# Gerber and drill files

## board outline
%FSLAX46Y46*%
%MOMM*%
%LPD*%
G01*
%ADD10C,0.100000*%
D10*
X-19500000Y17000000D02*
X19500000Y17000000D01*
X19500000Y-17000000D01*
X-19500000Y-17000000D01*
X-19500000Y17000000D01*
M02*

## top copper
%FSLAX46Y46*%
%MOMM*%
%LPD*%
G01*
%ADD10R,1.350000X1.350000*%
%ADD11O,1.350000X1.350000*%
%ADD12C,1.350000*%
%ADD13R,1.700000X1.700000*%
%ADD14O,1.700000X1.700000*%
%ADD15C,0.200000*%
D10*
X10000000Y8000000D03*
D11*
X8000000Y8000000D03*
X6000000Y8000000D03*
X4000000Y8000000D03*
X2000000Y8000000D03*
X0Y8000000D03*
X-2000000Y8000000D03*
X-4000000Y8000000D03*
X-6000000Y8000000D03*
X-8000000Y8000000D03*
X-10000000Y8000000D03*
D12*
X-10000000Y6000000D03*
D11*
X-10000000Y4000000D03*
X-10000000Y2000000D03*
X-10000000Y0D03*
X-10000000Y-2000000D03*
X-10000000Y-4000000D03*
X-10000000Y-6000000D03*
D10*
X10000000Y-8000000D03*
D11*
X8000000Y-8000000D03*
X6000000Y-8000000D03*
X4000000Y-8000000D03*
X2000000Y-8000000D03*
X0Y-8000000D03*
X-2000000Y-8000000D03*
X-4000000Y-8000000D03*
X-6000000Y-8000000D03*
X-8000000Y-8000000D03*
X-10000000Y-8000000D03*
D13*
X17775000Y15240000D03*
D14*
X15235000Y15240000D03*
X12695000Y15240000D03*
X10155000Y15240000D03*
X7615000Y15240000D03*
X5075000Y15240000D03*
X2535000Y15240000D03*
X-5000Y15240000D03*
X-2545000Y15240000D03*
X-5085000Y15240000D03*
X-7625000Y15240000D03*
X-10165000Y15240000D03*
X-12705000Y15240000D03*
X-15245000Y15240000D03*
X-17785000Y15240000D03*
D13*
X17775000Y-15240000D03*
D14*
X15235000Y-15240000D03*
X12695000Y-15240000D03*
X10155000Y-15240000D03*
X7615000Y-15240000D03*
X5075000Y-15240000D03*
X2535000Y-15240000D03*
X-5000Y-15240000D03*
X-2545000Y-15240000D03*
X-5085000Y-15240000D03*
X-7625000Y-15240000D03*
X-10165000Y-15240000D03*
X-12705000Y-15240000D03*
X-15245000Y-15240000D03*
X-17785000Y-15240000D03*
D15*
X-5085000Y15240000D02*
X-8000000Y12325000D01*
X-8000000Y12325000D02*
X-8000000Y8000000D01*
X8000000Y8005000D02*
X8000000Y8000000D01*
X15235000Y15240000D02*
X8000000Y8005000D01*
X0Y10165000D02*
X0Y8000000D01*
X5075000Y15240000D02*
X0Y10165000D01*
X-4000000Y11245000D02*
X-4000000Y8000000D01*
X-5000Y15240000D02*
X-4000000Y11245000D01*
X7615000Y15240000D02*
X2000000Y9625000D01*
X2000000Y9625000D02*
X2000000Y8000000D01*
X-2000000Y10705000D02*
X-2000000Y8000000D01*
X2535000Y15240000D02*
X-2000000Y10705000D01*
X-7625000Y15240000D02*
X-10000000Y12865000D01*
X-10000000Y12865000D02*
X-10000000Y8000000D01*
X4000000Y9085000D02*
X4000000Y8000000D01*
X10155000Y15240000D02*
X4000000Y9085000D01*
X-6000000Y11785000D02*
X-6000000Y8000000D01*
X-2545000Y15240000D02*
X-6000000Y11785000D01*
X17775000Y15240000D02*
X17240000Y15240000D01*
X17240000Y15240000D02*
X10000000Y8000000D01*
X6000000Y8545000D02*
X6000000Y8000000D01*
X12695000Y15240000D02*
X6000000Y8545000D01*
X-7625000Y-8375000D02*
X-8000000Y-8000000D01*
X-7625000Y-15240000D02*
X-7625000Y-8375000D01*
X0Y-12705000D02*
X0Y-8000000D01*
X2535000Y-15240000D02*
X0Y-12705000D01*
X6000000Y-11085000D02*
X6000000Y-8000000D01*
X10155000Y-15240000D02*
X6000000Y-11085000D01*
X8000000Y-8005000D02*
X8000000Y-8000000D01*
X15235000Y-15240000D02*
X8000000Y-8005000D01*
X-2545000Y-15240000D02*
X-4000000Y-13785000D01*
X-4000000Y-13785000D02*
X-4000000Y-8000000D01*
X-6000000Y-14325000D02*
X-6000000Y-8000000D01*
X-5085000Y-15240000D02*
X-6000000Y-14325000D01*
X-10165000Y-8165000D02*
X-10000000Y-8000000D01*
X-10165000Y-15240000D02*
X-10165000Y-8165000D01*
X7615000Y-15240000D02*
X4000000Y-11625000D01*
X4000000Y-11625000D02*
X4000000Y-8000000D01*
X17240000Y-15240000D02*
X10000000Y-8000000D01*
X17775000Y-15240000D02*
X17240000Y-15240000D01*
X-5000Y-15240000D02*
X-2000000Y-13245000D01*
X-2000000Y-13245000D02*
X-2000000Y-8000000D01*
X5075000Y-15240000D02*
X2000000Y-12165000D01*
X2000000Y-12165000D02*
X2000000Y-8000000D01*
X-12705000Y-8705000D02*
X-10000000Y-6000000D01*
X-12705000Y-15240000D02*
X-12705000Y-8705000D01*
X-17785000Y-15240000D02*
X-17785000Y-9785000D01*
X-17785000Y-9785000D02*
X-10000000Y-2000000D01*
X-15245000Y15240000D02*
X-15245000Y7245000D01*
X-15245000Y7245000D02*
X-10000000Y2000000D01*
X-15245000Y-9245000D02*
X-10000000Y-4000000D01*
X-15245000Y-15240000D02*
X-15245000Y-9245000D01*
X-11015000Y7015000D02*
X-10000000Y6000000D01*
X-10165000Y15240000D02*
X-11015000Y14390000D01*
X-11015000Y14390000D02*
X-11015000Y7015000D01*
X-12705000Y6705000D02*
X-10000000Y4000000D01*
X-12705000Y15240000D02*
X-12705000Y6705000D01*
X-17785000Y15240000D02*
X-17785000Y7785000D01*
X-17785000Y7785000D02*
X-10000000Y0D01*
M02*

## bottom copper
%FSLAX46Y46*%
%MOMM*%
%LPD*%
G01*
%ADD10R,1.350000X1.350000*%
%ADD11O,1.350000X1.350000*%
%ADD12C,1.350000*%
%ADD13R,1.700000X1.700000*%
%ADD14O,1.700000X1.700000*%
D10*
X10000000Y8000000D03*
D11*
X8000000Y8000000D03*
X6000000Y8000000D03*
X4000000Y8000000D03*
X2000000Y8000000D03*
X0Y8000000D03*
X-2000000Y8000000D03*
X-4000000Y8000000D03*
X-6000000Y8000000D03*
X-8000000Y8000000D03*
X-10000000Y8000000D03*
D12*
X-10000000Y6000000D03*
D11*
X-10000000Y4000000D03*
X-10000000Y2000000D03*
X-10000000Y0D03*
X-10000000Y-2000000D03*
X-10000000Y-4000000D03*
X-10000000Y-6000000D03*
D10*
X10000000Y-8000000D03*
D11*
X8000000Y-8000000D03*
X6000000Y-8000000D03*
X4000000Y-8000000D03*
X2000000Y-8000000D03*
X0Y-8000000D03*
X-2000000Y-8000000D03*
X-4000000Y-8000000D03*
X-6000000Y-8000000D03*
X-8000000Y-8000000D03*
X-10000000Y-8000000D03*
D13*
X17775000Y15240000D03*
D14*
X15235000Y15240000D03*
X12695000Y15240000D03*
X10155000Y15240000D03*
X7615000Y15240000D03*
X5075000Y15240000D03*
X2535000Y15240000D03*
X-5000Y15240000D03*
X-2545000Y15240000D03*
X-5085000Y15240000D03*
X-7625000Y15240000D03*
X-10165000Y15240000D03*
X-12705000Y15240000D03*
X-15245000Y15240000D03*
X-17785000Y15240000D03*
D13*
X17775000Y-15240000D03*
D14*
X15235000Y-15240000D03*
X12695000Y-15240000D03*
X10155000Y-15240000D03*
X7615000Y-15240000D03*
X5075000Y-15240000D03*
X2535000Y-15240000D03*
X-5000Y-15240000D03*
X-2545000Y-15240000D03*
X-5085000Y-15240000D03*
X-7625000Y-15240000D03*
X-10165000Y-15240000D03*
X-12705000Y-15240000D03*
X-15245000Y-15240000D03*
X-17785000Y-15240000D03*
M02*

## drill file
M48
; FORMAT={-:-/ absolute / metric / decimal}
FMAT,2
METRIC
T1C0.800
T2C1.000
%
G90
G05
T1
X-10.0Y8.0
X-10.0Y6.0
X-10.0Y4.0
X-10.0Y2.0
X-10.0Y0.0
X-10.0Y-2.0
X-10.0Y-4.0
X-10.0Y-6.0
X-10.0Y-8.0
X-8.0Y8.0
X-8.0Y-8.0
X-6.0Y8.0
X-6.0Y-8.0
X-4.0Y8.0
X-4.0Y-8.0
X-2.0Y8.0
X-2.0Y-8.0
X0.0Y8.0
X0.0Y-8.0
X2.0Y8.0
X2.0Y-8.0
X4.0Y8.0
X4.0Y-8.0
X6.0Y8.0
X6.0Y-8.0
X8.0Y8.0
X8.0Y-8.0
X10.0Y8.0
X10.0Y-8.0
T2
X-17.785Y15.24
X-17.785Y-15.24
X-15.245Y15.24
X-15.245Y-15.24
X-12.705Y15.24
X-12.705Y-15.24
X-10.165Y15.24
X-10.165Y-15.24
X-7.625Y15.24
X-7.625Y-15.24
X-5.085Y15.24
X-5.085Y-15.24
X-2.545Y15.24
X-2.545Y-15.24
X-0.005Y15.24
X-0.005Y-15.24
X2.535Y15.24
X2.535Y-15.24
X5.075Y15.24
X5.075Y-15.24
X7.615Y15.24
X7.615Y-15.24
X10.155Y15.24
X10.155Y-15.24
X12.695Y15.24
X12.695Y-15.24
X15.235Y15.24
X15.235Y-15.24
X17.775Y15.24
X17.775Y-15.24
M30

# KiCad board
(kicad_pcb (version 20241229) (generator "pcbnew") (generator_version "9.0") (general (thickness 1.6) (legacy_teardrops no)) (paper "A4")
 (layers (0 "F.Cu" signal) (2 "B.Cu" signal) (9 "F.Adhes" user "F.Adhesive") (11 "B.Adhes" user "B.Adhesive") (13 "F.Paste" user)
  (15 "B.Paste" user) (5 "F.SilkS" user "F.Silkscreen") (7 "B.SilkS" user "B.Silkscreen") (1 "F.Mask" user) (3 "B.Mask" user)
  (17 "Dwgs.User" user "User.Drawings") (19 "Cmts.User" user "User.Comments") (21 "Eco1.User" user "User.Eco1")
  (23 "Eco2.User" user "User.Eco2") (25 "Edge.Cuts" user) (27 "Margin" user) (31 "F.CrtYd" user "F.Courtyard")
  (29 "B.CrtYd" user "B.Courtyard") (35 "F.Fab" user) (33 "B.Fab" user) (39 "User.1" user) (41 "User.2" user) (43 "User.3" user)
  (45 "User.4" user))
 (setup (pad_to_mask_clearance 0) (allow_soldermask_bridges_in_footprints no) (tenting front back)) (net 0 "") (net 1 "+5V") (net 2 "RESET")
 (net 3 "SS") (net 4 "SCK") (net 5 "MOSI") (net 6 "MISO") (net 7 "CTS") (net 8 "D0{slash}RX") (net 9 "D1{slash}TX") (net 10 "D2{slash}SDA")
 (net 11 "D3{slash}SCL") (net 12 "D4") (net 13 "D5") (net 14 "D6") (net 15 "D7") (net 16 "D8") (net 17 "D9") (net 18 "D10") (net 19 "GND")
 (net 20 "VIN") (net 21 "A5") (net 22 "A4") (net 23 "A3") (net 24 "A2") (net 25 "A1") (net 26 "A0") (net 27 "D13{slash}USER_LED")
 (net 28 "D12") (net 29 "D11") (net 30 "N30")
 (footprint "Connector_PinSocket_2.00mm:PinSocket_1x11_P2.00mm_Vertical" (layer "F.Cu") (at 10 -8 -90)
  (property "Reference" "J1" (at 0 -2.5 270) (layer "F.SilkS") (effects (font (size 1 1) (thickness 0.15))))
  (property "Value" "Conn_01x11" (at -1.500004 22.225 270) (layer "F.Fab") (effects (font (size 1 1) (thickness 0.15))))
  (pad "1" thru_hole rect (at 0 0 270) (size 1.35 1.35) (drill 0.8) (layers "*.Cu" "*.Mask") (remove_unused_layers no) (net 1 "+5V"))
  (pad "2" thru_hole oval (at 0 2 270) (size 1.35 1.35) (drill 0.8) (layers "*.Cu" "*.Mask") (remove_unused_layers no) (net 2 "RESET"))
  (pad "3" thru_hole oval (at 0 4 270) (size 1.35 1.35) (drill 0.8) (layers "*.Cu" "*.Mask") (remove_unused_layers no) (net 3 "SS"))
  (pad "4" thru_hole oval (at 0 6 270) (size 1.35 1.35) (drill 0.8) (layers "*.Cu" "*.Mask") (remove_unused_layers no) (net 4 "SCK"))
  (pad "5" thru_hole oval (at 0 8 270) (size 1.35 1.35) (drill 0.8) (layers "*.Cu" "*.Mask") (remove_unused_layers no) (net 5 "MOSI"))
  (pad "6" thru_hole oval (at 0 10 270) (size 1.35 1.35) (drill 0.8) (layers "*.Cu" "*.Mask") (remove_unused_layers no) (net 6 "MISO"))
  (pad "7" thru_hole oval (at 0 12 270) (size 1.35 1.35) (drill 0.8) (layers "*.Cu" "*.Mask") (remove_unused_layers no) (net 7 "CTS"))
  (pad "8" thru_hole oval (at 0 14 270) (size 1.35 1.35) (drill 0.8) (layers "*.Cu" "*.Mask") (remove_unused_layers no)
   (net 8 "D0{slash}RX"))
  (pad "9" thru_hole oval (at 0 16 270) (size 1.35 1.35) (drill 0.8) (layers "*.Cu" "*.Mask") (remove_unused_layers no)
   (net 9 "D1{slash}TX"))
  (pad "10" thru_hole oval (at 0 18 270) (size 1.35 1.35) (drill 0.8) (layers "*.Cu" "*.Mask") (remove_unused_layers no)
   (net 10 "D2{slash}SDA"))
  (pad "11" thru_hole oval (at 0 20 270) (size 1.35 1.35) (drill 0.8) (layers "*.Cu" "*.Mask") (remove_unused_layers no)
   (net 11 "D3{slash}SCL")))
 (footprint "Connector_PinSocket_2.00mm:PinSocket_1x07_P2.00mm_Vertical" (layer "F.Cu") (at -10 -6)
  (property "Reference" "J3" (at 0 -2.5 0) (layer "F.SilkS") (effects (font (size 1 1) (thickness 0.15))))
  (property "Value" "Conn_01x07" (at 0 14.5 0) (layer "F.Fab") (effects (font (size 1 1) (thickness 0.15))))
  (pad "1" thru_hole circle (at 0 0) (size 1.35 1.35) (drill 0.8) (layers "*.Cu" "*.Mask") (remove_unused_layers no) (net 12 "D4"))
  (pad "2" thru_hole oval (at 0 2) (size 1.35 1.35) (drill 0.8) (layers "*.Cu" "*.Mask") (remove_unused_layers no) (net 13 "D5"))
  (pad "3" thru_hole oval (at 0 4) (size 1.35 1.35) (drill 0.8) (layers "*.Cu" "*.Mask") (remove_unused_layers no) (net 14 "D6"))
  (pad "4" thru_hole oval (at 0 6) (size 1.35 1.35) (drill 0.8) (layers "*.Cu" "*.Mask") (remove_unused_layers no) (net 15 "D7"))
  (pad "5" thru_hole oval (at 0 8) (size 1.35 1.35) (drill 0.8) (layers "*.Cu" "*.Mask") (remove_unused_layers no) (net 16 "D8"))
  (pad "6" thru_hole oval (at 0 10) (size 1.35 1.35) (drill 0.8) (layers "*.Cu" "*.Mask") (remove_unused_layers no) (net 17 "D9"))
  (pad "7" thru_hole oval (at 0 12) (size 1.35 1.35) (drill 0.8) (layers "*.Cu" "*.Mask") (remove_unused_layers no) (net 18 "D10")))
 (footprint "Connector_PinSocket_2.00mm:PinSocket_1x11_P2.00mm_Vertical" (layer "F.Cu") (at 10 8 -90)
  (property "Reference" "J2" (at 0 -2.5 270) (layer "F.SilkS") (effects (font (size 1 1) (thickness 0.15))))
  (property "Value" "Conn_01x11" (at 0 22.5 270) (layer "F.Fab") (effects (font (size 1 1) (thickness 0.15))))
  (pad "1" thru_hole rect (at 0 0 270) (size 1.35 1.35) (drill 0.8) (layers "*.Cu" "*.Mask") (remove_unused_layers no) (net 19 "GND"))
  (pad "2" thru_hole oval (at 0 2 270) (size 1.35 1.35) (drill 0.8) (layers "*.Cu" "*.Mask") (remove_unused_layers no) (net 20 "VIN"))
  (pad "3" thru_hole oval (at 0 4 270) (size 1.35 1.35) (drill 0.8) (layers "*.Cu" "*.Mask") (remove_unused_layers no) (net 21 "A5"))
  (pad "4" thru_hole oval (at 0 6 270) (size 1.35 1.35) (drill 0.8) (layers "*.Cu" "*.Mask") (remove_unused_layers no) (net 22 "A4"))
  (pad "5" thru_hole oval (at 0 8 270) (size 1.35 1.35) (drill 0.8) (layers "*.Cu" "*.Mask") (remove_unused_layers no) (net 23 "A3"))
  (pad "6" thru_hole oval (at 0 10 270) (size 1.35 1.35) (drill 0.8) (layers "*.Cu" "*.Mask") (remove_unused_layers no) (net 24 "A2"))
  (pad "7" thru_hole oval (at 0 12 270) (size 1.35 1.35) (drill 0.8) (layers "*.Cu" "*.Mask") (remove_unused_layers no) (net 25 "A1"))
  (pad "8" thru_hole oval (at 0 14 270) (size 1.35 1.35) (drill 0.8) (layers "*.Cu" "*.Mask") (remove_unused_layers no) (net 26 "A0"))
  (pad "9" thru_hole oval (at 0 16 270) (size 1.35 1.35) (drill 0.8) (layers "*.Cu" "*.Mask") (remove_unused_layers no)
   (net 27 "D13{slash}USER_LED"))
  (pad "10" thru_hole oval (at 0 18 270) (size 1.35 1.35) (drill 0.8) (layers "*.Cu" "*.Mask") (remove_unused_layers no) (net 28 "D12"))
  (pad "11" thru_hole oval (at 0 20 270) (size 1.35 1.35) (drill 0.8) (layers "*.Cu" "*.Mask") (remove_unused_layers no) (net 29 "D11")))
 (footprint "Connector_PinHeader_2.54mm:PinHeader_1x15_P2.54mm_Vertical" (layer "B.Cu") (at 17.775 -15.24 90)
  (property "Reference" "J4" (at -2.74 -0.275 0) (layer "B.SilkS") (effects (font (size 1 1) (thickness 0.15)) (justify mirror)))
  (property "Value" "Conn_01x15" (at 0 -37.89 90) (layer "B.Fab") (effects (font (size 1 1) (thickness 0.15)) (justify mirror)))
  (pad "1" thru_hole rect (at 0 0 90) (size 1.7 1.7) (drill 1) (layers "*.Cu" "*.Mask") (remove_unused_layers no) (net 1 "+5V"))
  (pad "2" thru_hole oval (at 0 -2.54 90) (size 1.7 1.7) (drill 1) (layers "*.Cu" "*.Mask") (remove_unused_layers no) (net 2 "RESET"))
  (pad "3" thru_hole oval (at 0 -5.08 90) (size 1.7 1.7) (drill 1) (layers "*.Cu" "*.Mask") (remove_unused_layers no) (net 3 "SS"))
  (pad "4" thru_hole oval (at 0 -7.62 90) (size 1.7 1.7) (drill 1) (layers "*.Cu" "*.Mask") (remove_unused_layers no) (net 4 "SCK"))
  (pad "5" thru_hole oval (at 0 -10.16 90) (size 1.7 1.7) (drill 1) (layers "*.Cu" "*.Mask") (remove_unused_layers no) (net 5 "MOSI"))
  (pad "6" thru_hole oval (at 0 -12.7 90) (size 1.7 1.7) (drill 1) (layers "*.Cu" "*.Mask") (remove_unused_layers no) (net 6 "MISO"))
  (pad "7" thru_hole oval (at 0 -15.24 90) (size 1.7 1.7) (drill 1) (layers "*.Cu" "*.Mask") (remove_unused_layers no) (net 7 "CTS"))
  (pad "8" thru_hole oval (at 0 -17.78 90) (size 1.7 1.7) (drill 1) (layers "*.Cu" "*.Mask") (remove_unused_layers no) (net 8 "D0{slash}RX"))
  (pad "9" thru_hole oval (at 0 -20.32 90) (size 1.7 1.7) (drill 1) (layers "*.Cu" "*.Mask") (remove_unused_layers no) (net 9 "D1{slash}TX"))
  (pad "10" thru_hole oval (at 0 -22.86 90) (size 1.7 1.7) (drill 1) (layers "*.Cu" "*.Mask") (remove_unused_layers no)
   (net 10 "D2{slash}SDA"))
  (pad "11" thru_hole oval (at 0 -25.4 90) (size 1.7 1.7) (drill 1) (layers "*.Cu" "*.Mask") (remove_unused_layers no)
   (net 11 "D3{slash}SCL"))
  (pad "12" thru_hole oval (at 0 -27.94 90) (size 1.7 1.7) (drill 1) (layers "*.Cu" "*.Mask") (remove_unused_layers no) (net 12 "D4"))
  (pad "13" thru_hole oval (at 0 -30.48 90) (size 1.7 1.7) (drill 1) (layers "*.Cu" "*.Mask") (remove_unused_layers no) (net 13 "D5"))
  (pad "14" thru_hole oval (at 0 -33.02 90) (size 1.7 1.7) (drill 1) (layers "*.Cu" "*.Mask") (remove_unused_layers no) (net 14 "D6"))
  (pad "15" thru_hole oval (at 0 -35.56 90) (size 1.7 1.7) (drill 1) (layers "*.Cu" "*.Mask") (remove_unused_layers no) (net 15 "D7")))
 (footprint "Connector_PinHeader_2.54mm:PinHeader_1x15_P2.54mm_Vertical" (layer "B.Cu") (at 17.775 15.24 90)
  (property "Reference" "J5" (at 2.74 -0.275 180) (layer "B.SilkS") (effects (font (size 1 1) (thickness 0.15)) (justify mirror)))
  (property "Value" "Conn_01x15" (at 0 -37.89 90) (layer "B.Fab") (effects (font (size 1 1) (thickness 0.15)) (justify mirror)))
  (pad "1" thru_hole rect (at 0 0 90) (size 1.7 1.7) (drill 1) (layers "*.Cu" "*.Mask") (remove_unused_layers no) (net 19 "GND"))
  (pad "2" thru_hole oval (at 0 -2.54 90) (size 1.7 1.7) (drill 1) (layers "*.Cu" "*.Mask") (remove_unused_layers no) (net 20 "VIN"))
  (pad "3" thru_hole oval (at 0 -5.08 90) (size 1.7 1.7) (drill 1) (layers "*.Cu" "*.Mask") (remove_unused_layers no) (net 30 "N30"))
  (pad "4" thru_hole oval (at 0 -7.62 90) (size 1.7 1.7) (drill 1) (layers "*.Cu" "*.Mask") (remove_unused_layers no) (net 21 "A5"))
  (pad "5" thru_hole oval (at 0 -10.16 90) (size 1.7 1.7) (drill 1) (layers "*.Cu" "*.Mask") (remove_unused_layers no) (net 22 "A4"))
  (pad "6" thru_hole oval (at 0 -12.7 90) (size 1.7 1.7) (drill 1) (layers "*.Cu" "*.Mask") (remove_unused_layers no) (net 23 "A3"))
  (pad "7" thru_hole oval (at 0 -15.24 90) (size 1.7 1.7) (drill 1) (layers "*.Cu" "*.Mask") (remove_unused_layers no) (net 24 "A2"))
  (pad "8" thru_hole oval (at 0 -17.78 90) (size 1.7 1.7) (drill 1) (layers "*.Cu" "*.Mask") (remove_unused_layers no) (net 25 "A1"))
  (pad "9" thru_hole oval (at 0 -20.32 90) (size 1.7 1.7) (drill 1) (layers "*.Cu" "*.Mask") (remove_unused_layers no) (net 26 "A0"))
  (pad "10" thru_hole oval (at 0 -22.86 90) (size 1.7 1.7) (drill 1) (layers "*.Cu" "*.Mask") (remove_unused_layers no)
   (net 27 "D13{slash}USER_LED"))
  (pad "11" thru_hole oval (at 0 -25.4 90) (size 1.7 1.7) (drill 1) (layers "*.Cu" "*.Mask") (remove_unused_layers no) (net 28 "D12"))
  (pad "12" thru_hole oval (at 0 -27.94 90) (size 1.7 1.7) (drill 1) (layers "*.Cu" "*.Mask") (remove_unused_layers no) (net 29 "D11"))
  (pad "13" thru_hole oval (at 0 -30.48 90) (size 1.7 1.7) (drill 1) (layers "*.Cu" "*.Mask") (remove_unused_layers no) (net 18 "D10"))
  (pad "14" thru_hole oval (at 0 -33.02 90) (size 1.7 1.7) (drill 1) (layers "*.Cu" "*.Mask") (remove_unused_layers no) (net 17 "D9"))
  (pad "15" thru_hole oval (at 0 -35.56 90) (size 1.7 1.7) (drill 1) (layers "*.Cu" "*.Mask") (remove_unused_layers no) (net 16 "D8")))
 (gr_rect (start -19.5 -17) (end 19.5 17) (stroke (width 0.1) (type solid)) (fill no) (layer "Edge.Cuts"))
 (segment (start -5.085 -15.24) (end -8 -12.325) (width 0.2) (layer "F.Cu") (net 10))
 (segment (start -8 -12.325) (end -8 -8) (width 0.2) (layer "F.Cu") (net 10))
 (segment (start 8 -8.005) (end 8 -8) (width 0.2) (layer "F.Cu") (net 2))
 (segment (start 15.235 -15.24) (end 8 -8.005) (width 0.2) (layer "F.Cu") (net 2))
 (segment (start 0 -10.165) (end 0 -8) (width 0.2) (layer "F.Cu") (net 6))
 (segment (start 5.075 -15.24) (end 0 -10.165) (width 0.2) (layer "F.Cu") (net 6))
 (segment (start -4 -11.245) (end -4 -8) (width 0.2) (layer "F.Cu") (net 8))
 (segment (start -0.005 -15.24) (end -4 -11.245) (width 0.2) (layer "F.Cu") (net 8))
 (segment (start 7.615 -15.24) (end 2 -9.625) (width 0.2) (layer "F.Cu") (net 5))
 (segment (start 2 -9.625) (end 2 -8) (width 0.2) (layer "F.Cu") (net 5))
 (segment (start -2 -10.705) (end -2 -8) (width 0.2) (layer "F.Cu") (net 7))
 (segment (start 2.535 -15.24) (end -2 -10.705) (width 0.2) (layer "F.Cu") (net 7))
 (segment (start -7.625 -15.24) (end -10 -12.865) (width 0.2) (layer "F.Cu") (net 11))
 (segment (start -10 -12.865) (end -10 -8) (width 0.2) (layer "F.Cu") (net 11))
 (segment (start 4 -9.085) (end 4 -8) (width 0.2) (layer "F.Cu") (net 4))
 (segment (start 10.155 -15.24) (end 4 -9.085) (width 0.2) (layer "F.Cu") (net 4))
 (segment (start -6 -11.785) (end -6 -8) (width 0.2) (layer "F.Cu") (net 9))
 (segment (start -2.545 -15.24) (end -6 -11.785) (width 0.2) (layer "F.Cu") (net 9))
 (segment (start 17.775 -15.24) (end 17.24 -15.24) (width 0.2) (layer "F.Cu") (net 1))
 (segment (start 17.24 -15.24) (end 10 -8) (width 0.2) (layer "F.Cu") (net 1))
 (segment (start 6 -8.545) (end 6 -8) (width 0.2) (layer "F.Cu") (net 3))
 (segment (start 12.695 -15.24) (end 6 -8.545) (width 0.2) (layer "F.Cu") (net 3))
 (segment (start -7.625 8.375) (end -8 8) (width 0.2) (layer "F.Cu") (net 28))
 (segment (start -7.625 15.24) (end -7.625 8.375) (width 0.2) (layer "F.Cu") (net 28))
 (segment (start 0 12.705) (end 0 8) (width 0.2) (layer "F.Cu") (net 24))
 (segment (start 2.535 15.24) (end 0 12.705) (width 0.2) (layer "F.Cu") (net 24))
 (segment (start 6 11.085) (end 6 8) (width 0.2) (layer "F.Cu") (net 21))
 (segment (start 10.155 15.24) (end 6 11.085) (width 0.2) (layer "F.Cu") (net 21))
 (segment (start 8 8.005) (end 8 8) (width 0.2) (layer "F.Cu") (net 20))
 (segment (start 15.235 15.24) (end 8 8.005) (width 0.2) (layer "F.Cu") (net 20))
 (segment (start -2.545 15.24) (end -4 13.785) (width 0.2) (layer "F.Cu") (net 26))
 (segment (start -4 13.785) (end -4 8) (width 0.2) (layer "F.Cu") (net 26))
 (segment (start -6 14.325) (end -6 8) (width 0.2) (layer "F.Cu") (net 27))
 (segment (start -5.085 15.24) (end -6 14.325) (width 0.2) (layer "F.Cu") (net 27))
 (segment (start -10.165 8.165) (end -10 8) (width 0.2) (layer "F.Cu") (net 29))
 (segment (start -10.165 15.24) (end -10.165 8.165) (width 0.2) (layer "F.Cu") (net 29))
 (segment (start 7.615 15.24) (end 4 11.625) (width 0.2) (layer "F.Cu") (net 22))
 (segment (start 4 11.625) (end 4 8) (width 0.2) (layer "F.Cu") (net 22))
 (segment (start 17.24 15.24) (end 10 8) (width 0.2) (layer "F.Cu") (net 19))
 (segment (start 17.775 15.24) (end 17.24 15.24) (width 0.2) (layer "F.Cu") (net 19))
 (segment (start -0.005 15.24) (end -2 13.245) (width 0.2) (layer "F.Cu") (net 25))
 (segment (start -2 13.245) (end -2 8) (width 0.2) (layer "F.Cu") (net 25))
 (segment (start 5.075 15.24) (end 2 12.165) (width 0.2) (layer "F.Cu") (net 23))
 (segment (start 2 12.165) (end 2 8) (width 0.2) (layer "F.Cu") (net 23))
 (segment (start -12.705 8.705) (end -10 6) (width 0.2) (layer "F.Cu") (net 18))
 (segment (start -12.705 15.24) (end -12.705 8.705) (width 0.2) (layer "F.Cu") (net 18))
 (segment (start -17.785 15.24) (end -17.785 9.785) (width 0.2) (layer "F.Cu") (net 16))
 (segment (start -17.785 9.785) (end -10 2) (width 0.2) (layer "F.Cu") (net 16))
 (segment (start -15.245 -15.24) (end -15.245 -7.245) (width 0.2) (layer "F.Cu") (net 14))
 (segment (start -15.245 -7.245) (end -10 -2) (width 0.2) (layer "F.Cu") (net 14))
 (segment (start -15.245 9.245) (end -10 4) (width 0.2) (layer "F.Cu") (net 17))
 (segment (start -15.245 15.24) (end -15.245 9.245) (width 0.2) (layer "F.Cu") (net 17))
 (segment (start -11.015 -7.015) (end -10 -6) (width 0.2) (layer "F.Cu") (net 12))
 (segment (start -10.165 -15.24) (end -11.015 -14.39) (width 0.2) (layer "F.Cu") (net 12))
 (segment (start -11.015 -14.39) (end -11.015 -7.015) (width 0.2) (layer "F.Cu") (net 12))
 (segment (start -12.705 -6.705) (end -10 -4) (width 0.2) (layer "F.Cu") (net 13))
 (segment (start -12.705 -15.24) (end -12.705 -6.705) (width 0.2) (layer "F.Cu") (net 13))
 (segment (start -17.785 -15.24) (end -17.785 -7.785) (width 0.2) (layer "F.Cu") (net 15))
 (segment (start -17.785 -7.785) (end -10 0) (width 0.2) (layer "F.Cu") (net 15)))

